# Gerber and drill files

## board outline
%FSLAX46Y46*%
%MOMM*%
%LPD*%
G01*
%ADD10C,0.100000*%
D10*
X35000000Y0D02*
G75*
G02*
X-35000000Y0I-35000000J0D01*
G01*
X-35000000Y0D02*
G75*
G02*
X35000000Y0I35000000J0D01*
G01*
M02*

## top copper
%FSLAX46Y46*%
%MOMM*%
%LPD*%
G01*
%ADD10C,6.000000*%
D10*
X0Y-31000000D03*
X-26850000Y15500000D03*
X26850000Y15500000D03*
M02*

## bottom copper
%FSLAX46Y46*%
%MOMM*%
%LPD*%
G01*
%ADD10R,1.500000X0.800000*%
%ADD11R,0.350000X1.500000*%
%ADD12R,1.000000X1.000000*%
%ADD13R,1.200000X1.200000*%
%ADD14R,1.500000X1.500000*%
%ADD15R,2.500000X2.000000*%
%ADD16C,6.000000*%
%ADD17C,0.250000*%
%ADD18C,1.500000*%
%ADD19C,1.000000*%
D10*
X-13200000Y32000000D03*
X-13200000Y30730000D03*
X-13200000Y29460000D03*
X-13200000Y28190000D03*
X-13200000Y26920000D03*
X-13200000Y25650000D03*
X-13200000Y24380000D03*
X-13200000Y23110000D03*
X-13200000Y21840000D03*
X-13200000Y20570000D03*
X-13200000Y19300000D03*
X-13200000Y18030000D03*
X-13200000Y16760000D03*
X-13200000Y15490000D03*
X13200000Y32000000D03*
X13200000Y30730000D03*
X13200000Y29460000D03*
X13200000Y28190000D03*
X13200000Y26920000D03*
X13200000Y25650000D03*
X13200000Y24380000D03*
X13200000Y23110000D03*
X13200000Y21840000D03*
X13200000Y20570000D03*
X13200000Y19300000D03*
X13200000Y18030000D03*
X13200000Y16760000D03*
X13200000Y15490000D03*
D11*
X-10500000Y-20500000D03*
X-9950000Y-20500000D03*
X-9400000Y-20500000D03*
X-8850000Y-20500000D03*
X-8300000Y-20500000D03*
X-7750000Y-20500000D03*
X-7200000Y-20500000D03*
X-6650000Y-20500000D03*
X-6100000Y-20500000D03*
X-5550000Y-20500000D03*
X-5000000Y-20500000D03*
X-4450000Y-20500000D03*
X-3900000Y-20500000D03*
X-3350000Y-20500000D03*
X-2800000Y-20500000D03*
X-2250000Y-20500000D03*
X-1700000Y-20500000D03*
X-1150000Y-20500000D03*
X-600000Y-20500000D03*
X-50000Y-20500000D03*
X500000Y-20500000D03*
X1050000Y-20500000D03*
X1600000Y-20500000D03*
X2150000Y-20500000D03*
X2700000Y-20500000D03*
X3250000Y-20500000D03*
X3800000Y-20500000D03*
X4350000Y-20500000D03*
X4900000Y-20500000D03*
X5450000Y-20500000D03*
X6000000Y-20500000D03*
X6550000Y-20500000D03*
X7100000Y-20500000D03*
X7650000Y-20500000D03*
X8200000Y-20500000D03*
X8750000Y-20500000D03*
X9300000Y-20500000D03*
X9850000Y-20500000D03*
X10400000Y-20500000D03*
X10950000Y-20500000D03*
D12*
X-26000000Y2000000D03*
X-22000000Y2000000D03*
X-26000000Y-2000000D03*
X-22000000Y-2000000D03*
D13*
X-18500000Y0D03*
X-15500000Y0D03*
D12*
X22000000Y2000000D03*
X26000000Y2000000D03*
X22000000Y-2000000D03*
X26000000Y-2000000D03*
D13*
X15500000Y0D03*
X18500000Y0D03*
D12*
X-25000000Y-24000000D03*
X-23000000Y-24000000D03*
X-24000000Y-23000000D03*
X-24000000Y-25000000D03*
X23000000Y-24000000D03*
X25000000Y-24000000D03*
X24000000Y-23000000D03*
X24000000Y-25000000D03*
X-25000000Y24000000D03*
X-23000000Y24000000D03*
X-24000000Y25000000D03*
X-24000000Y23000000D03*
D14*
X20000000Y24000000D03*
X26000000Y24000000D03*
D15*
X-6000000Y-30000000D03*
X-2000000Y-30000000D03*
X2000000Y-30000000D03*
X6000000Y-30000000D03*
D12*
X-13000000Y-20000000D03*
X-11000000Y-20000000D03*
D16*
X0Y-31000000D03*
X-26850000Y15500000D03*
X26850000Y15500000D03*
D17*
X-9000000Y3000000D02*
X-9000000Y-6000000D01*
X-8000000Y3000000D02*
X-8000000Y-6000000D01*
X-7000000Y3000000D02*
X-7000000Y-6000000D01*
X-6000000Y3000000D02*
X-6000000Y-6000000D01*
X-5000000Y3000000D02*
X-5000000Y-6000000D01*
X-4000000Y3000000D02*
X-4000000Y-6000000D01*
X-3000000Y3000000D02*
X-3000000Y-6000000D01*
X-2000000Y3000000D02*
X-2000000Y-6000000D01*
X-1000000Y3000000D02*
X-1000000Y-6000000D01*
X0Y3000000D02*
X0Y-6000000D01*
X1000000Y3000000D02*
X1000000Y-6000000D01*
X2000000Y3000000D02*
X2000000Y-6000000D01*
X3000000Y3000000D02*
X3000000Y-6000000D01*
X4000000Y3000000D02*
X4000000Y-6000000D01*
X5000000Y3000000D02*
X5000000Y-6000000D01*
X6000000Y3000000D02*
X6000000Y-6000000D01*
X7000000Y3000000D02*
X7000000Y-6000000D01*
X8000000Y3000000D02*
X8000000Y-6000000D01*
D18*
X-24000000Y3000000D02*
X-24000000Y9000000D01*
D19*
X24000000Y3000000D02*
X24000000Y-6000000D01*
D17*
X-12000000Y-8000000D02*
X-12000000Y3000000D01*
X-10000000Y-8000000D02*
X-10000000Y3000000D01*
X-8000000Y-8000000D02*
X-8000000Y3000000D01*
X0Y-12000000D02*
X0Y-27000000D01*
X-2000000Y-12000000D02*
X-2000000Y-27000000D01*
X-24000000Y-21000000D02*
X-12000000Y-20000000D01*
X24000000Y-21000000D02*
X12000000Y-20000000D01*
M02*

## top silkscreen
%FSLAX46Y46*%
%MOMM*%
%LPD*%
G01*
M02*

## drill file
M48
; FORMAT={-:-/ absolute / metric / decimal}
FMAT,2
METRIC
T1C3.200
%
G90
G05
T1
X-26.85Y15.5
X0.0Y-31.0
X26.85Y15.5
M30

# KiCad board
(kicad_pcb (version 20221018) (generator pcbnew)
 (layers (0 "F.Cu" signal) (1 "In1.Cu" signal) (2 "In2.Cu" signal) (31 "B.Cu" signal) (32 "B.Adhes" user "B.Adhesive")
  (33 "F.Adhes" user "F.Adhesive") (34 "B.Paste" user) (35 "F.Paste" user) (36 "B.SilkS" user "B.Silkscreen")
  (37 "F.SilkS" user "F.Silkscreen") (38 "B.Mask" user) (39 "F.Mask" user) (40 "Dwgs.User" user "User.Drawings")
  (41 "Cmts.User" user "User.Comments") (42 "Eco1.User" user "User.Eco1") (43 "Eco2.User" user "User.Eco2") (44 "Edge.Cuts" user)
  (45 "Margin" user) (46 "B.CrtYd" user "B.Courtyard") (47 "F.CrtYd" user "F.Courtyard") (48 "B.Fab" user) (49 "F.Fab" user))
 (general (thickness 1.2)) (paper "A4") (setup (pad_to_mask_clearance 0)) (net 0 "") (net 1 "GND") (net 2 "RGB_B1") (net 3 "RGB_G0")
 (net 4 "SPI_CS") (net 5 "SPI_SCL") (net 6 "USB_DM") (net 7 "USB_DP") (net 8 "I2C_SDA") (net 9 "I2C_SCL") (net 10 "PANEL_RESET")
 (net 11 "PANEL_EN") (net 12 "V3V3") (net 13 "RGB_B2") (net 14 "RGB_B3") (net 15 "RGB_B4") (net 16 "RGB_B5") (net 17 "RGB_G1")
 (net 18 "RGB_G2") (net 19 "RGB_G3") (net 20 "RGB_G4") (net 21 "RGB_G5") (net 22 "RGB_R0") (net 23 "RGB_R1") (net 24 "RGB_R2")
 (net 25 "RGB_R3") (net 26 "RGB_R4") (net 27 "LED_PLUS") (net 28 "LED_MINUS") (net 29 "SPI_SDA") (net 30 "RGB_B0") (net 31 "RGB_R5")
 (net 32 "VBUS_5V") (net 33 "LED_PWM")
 (gr_circle (center 0 0) (end 35 0) (stroke (width 0.1) (type solid)) (fill none) (layer "Edge.Cuts"))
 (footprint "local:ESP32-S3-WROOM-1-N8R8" (layer "B.Cu") (at 0 -12 0)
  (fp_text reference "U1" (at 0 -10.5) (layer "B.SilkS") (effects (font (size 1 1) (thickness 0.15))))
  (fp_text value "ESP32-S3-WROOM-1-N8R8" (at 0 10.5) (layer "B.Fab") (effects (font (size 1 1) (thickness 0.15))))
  (pad "1" smd rect (at -13.2 -20.0) (size 1.5 0.8) (layers "B.Cu" "B.Mask" "B.Paste") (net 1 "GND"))
  (pad "2" smd rect (at -13.2 -18.73) (size 1.5 0.8) (layers "B.Cu" "B.Mask" "B.Paste") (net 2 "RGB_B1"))
  (pad "3" smd rect (at -13.2 -17.46) (size 1.5 0.8) (layers "B.Cu" "B.Mask" "B.Paste") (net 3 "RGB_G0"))
  (pad "4" smd rect (at -13.2 -16.19) (size 1.5 0.8) (layers "B.Cu" "B.Mask" "B.Paste") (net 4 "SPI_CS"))
  (pad "5" smd rect (at -13.2 -14.92) (size 1.5 0.8) (layers "B.Cu" "B.Mask" "B.Paste") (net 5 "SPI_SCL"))
  (pad "6" smd rect (at -13.2 -13.65) (size 1.5 0.8) (layers "B.Cu" "B.Mask" "B.Paste") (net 1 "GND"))
  (pad "7" smd rect (at -13.2 -12.379999999999999) (size 1.5 0.8) (layers "B.Cu" "B.Mask" "B.Paste") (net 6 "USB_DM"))
  (pad "8" smd rect (at -13.2 -11.11) (size 1.5 0.8) (layers "B.Cu" "B.Mask" "B.Paste") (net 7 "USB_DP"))
  (pad "9" smd rect (at -13.2 -9.84) (size 1.5 0.8) (layers "B.Cu" "B.Mask" "B.Paste") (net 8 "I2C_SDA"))
  (pad "10" smd rect (at -13.2 -8.57) (size 1.5 0.8) (layers "B.Cu" "B.Mask" "B.Paste") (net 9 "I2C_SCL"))
  (pad "11" smd rect (at -13.2 -7.300000000000001) (size 1.5 0.8) (layers "B.Cu" "B.Mask" "B.Paste") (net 1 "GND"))
  (pad "12" smd rect (at -13.2 -6.029999999999999) (size 1.5 0.8) (layers "B.Cu" "B.Mask" "B.Paste") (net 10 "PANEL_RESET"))
  (pad "13" smd rect (at -13.2 -4.76) (size 1.5 0.8) (layers "B.Cu" "B.Mask" "B.Paste") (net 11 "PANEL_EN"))
  (pad "14" smd rect (at -13.2 -3.4899999999999984) (size 1.5 0.8) (layers "B.Cu" "B.Mask" "B.Paste") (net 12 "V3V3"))
  (pad "15" smd rect (at 13.2 -20.0) (size 1.5 0.8) (layers "B.Cu" "B.Mask" "B.Paste") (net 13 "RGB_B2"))
  (pad "16" smd rect (at 13.2 -18.73) (size 1.5 0.8) (layers "B.Cu" "B.Mask" "B.Paste") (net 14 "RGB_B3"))
  (pad "17" smd rect (at 13.2 -17.46) (size 1.5 0.8) (layers "B.Cu" "B.Mask" "B.Paste") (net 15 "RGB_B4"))
  (pad "18" smd rect (at 13.2 -16.19) (size 1.5 0.8) (layers "B.Cu" "B.Mask" "B.Paste") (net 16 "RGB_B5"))
  (pad "19" smd rect (at 13.2 -14.92) (size 1.5 0.8) (layers "B.Cu" "B.Mask" "B.Paste") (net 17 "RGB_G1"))
  (pad "20" smd rect (at 13.2 -13.65) (size 1.5 0.8) (layers "B.Cu" "B.Mask" "B.Paste") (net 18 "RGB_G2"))
  (pad "21" smd rect (at 13.2 -12.379999999999999) (size 1.5 0.8) (layers "B.Cu" "B.Mask" "B.Paste") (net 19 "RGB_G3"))
  (pad "22" smd rect (at 13.2 -11.11) (size 1.5 0.8) (layers "B.Cu" "B.Mask" "B.Paste") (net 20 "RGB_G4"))
  (pad "23" smd rect (at 13.2 -9.84) (size 1.5 0.8) (layers "B.Cu" "B.Mask" "B.Paste") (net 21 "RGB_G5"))
  (pad "24" smd rect (at 13.2 -8.57) (size 1.5 0.8) (layers "B.Cu" "B.Mask" "B.Paste") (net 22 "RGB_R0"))
  (pad "25" smd rect (at 13.2 -7.300000000000001) (size 1.5 0.8) (layers "B.Cu" "B.Mask" "B.Paste") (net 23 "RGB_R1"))
  (pad "26" smd rect (at 13.2 -6.029999999999999) (size 1.5 0.8) (layers "B.Cu" "B.Mask" "B.Paste") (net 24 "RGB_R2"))
  (pad "27" smd rect (at 13.2 -4.76) (size 1.5 0.8) (layers "B.Cu" "B.Mask" "B.Paste") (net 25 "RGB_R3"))
  (pad "28" smd rect (at 13.2 -3.4899999999999984) (size 1.5 0.8) (layers "B.Cu" "B.Mask" "B.Paste") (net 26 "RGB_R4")))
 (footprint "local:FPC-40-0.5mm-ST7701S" (layer "B.Cu") (at 0 8 0)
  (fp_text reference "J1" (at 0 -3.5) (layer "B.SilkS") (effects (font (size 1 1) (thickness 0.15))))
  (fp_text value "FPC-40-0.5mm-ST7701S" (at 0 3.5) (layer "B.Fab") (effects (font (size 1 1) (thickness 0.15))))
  (pad "1" smd rect (at -10.5 12.5) (size 0.35 1.5) (layers "B.Cu" "B.Mask" "B.Paste") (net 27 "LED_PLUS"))
  (pad "2" smd rect (at -9.95 12.5) (size 0.35 1.5) (layers "B.Cu" "B.Mask" "B.Paste") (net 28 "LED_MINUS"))
  (pad "3" smd rect (at -9.4 12.5) (size 0.35 1.5) (layers "B.Cu" "B.Mask" "B.Paste") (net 1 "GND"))
  (pad "4" smd rect (at -8.85 12.5) (size 0.35 1.5) (layers "B.Cu" "B.Mask" "B.Paste") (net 12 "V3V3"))
  (pad "5" smd rect (at -8.3 12.5) (size 0.35 1.5) (layers "B.Cu" "B.Mask" "B.Paste") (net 10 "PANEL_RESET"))
  (pad "6" smd rect (at -7.75 12.5) (size 0.35 1.5) (layers "B.Cu" "B.Mask" "B.Paste") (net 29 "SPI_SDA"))
  (pad "7" smd rect (at -7.199999999999999 12.5) (size 0.35 1.5) (layers "B.Cu" "B.Mask" "B.Paste") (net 5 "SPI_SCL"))
  (pad "8" smd rect (at -6.6499999999999995 12.5) (size 0.35 1.5) (layers "B.Cu" "B.Mask" "B.Paste") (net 4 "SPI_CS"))
  (pad "9" smd rect (at -6.1 12.5) (size 0.35 1.5) (layers "B.Cu" "B.Mask" "B.Paste") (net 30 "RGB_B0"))
  (pad "10" smd rect (at -5.55 12.5) (size 0.35 1.5) (layers "B.Cu" "B.Mask" "B.Paste") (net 2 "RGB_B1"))
  (pad "11" smd rect (at -5.0 12.5) (size 0.35 1.5) (layers "B.Cu" "B.Mask" "B.Paste") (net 13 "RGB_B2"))
  (pad "12" smd rect (at -4.449999999999999 12.5) (size 0.35 1.5) (layers "B.Cu" "B.Mask" "B.Paste") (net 14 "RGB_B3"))
  (pad "13" smd rect (at -3.8999999999999995 12.5) (size 0.35 1.5) (layers "B.Cu" "B.Mask" "B.Paste") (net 15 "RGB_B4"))
  (pad "14" smd rect (at -3.3499999999999996 12.5) (size 0.35 1.5) (layers "B.Cu" "B.Mask" "B.Paste") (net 16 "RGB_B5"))
  (pad "15" smd rect (at -2.799999999999999 12.5) (size 0.35 1.5) (layers "B.Cu" "B.Mask" "B.Paste") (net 3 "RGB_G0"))
  (pad "16" smd rect (at -2.25 12.5) (size 0.35 1.5) (layers "B.Cu" "B.Mask" "B.Paste") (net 17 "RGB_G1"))
  (pad "17" smd rect (at -1.6999999999999993 12.5) (size 0.35 1.5) (layers "B.Cu" "B.Mask" "B.Paste") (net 18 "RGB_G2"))
  (pad "18" smd rect (at -1.1499999999999986 12.5) (size 0.35 1.5) (layers "B.Cu" "B.Mask" "B.Paste") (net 19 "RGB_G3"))
  (pad "19" smd rect (at -0.5999999999999996 12.5) (size 0.35 1.5) (layers "B.Cu" "B.Mask" "B.Paste") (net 20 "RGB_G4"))
  (pad "20" smd rect (at -0.049999999999998934 12.5) (size 0.35 1.5) (layers "B.Cu" "B.Mask" "B.Paste") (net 21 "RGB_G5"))
  (pad "21" smd rect (at 0.5 12.5) (size 0.35 1.5) (layers "B.Cu" "B.Mask" "B.Paste") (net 22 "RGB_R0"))
  (pad "22" smd rect (at 1.0500000000000007 12.5) (size 0.35 1.5) (layers "B.Cu" "B.Mask" "B.Paste") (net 23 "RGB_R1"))
  (pad "23" smd rect (at 1.6000000000000014 12.5) (size 0.35 1.5) (layers "B.Cu" "B.Mask" "B.Paste") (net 24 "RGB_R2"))
  (pad "24" smd rect (at 2.1500000000000004 12.5) (size 0.35 1.5) (layers "B.Cu" "B.Mask" "B.Paste") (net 25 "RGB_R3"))
  (pad "25" smd rect (at 2.700000000000001 12.5) (size 0.35 1.5) (layers "B.Cu" "B.Mask" "B.Paste") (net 26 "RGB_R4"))
  (pad "26" smd rect (at 3.2500000000000018 12.5) (size 0.35 1.5) (layers "B.Cu" "B.Mask" "B.Paste") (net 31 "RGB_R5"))
  (pad "27" smd rect (at 3.8000000000000007 12.5) (size 0.35 1.5) (layers "B.Cu" "B.Mask" "B.Paste") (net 1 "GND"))
  (pad "28" smd rect (at 4.350000000000001 12.5) (size 0.35 1.5) (layers "B.Cu" "B.Mask" "B.Paste") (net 1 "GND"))
  (pad "29" smd rect (at 4.900000000000002 12.5) (size 0.35 1.5) (layers "B.Cu" "B.Mask" "B.Paste") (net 1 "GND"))
  (pad "30" smd rect (at 5.450000000000001 12.5) (size 0.35 1.5) (layers "B.Cu" "B.Mask" "B.Paste") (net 1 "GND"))
  (pad "31" smd rect (at 6.0 12.5) (size 0.35 1.5) (layers "B.Cu" "B.Mask" "B.Paste") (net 1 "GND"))
  (pad "32" smd rect (at 6.550000000000001 12.5) (size 0.35 1.5) (layers "B.Cu" "B.Mask" "B.Paste") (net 1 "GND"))
  (pad "33" smd rect (at 7.100000000000001 12.5) (size 0.35 1.5) (layers "B.Cu" "B.Mask" "B.Paste") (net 1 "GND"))
  (pad "34" smd rect (at 7.650000000000002 12.5) (size 0.35 1.5) (layers "B.Cu" "B.Mask" "B.Paste") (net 1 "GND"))
  (pad "35" smd rect (at 8.200000000000003 12.5) (size 0.35 1.5) (layers "B.Cu" "B.Mask" "B.Paste") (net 1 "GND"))
  (pad "36" smd rect (at 8.75 12.5) (size 0.35 1.5) (layers "B.Cu" "B.Mask" "B.Paste") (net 1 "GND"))
  (pad "37" smd rect (at 9.3 12.5) (size 0.35 1.5) (layers "B.Cu" "B.Mask" "B.Paste") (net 1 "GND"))
  (pad "38" smd rect (at 9.850000000000001 12.5) (size 0.35 1.5) (layers "B.Cu" "B.Mask" "B.Paste") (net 1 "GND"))
  (pad "39" smd rect (at 10.400000000000002 12.5) (size 0.35 1.5) (layers "B.Cu" "B.Mask" "B.Paste") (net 1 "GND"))
  (pad "40" smd rect (at 10.950000000000003 12.5) (size 0.35 1.5) (layers "B.Cu" "B.Mask" "B.Paste") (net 1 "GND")))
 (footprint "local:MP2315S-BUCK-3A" (layer "B.Cu") (at -24 0 0)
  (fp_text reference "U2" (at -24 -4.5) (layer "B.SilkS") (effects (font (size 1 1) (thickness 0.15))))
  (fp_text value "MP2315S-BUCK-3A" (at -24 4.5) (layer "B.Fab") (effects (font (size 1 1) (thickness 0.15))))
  (pad "1" smd rect (at -2 -2) (size 1 1) (layers "B.Cu" "B.Mask" "B.Paste") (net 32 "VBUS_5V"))
  (pad "2" smd rect (at 2 -2) (size 1 1) (layers "B.Cu" "B.Mask" "B.Paste") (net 12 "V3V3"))
  (pad "3" smd rect (at -2 2) (size 1 1) (layers "B.Cu" "B.Mask" "B.Paste") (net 1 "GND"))
  (pad "4" smd rect (at 2 2) (size 1 1) (layers "B.Cu" "B.Mask" "B.Paste") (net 12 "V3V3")))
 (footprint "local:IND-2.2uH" (layer "B.Cu") (at -17 0 0)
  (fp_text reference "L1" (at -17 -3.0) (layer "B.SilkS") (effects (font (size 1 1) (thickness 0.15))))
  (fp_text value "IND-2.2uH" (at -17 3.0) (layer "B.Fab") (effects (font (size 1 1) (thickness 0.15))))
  (pad "1" smd rect (at -1.5 0) (size 1.2 1.2) (layers "B.Cu" "B.Mask" "B.Paste") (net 12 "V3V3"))
  (pad "2" smd rect (at 1.5 0) (size 1.2 1.2) (layers "B.Cu" "B.Mask" "B.Paste") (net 12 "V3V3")))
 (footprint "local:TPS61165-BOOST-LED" (layer "B.Cu") (at 24 0 0)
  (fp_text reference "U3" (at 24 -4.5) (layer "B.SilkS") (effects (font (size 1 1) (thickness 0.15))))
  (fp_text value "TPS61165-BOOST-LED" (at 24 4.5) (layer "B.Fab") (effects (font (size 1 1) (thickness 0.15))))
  (pad "1" smd rect (at -2 -2) (size 1 1) (layers "B.Cu" "B.Mask" "B.Paste") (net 32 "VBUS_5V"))
  (pad "2" smd rect (at 2 -2) (size 1 1) (layers "B.Cu" "B.Mask" "B.Paste") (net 27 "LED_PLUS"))
  (pad "3" smd rect (at -2 2) (size 1 1) (layers "B.Cu" "B.Mask" "B.Paste") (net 1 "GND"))
  (pad "4" smd rect (at 2 2) (size 1 1) (layers "B.Cu" "B.Mask" "B.Paste") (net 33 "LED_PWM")))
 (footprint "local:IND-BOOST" (layer "B.Cu") (at 17 0 0)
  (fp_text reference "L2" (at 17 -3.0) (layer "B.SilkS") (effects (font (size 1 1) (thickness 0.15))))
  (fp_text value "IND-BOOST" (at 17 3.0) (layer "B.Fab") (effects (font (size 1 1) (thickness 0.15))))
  (pad "1" smd rect (at -1.5 0) (size 1.2 1.2) (layers "B.Cu" "B.Mask" "B.Paste") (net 32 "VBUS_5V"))
  (pad "2" smd rect (at 1.5 0) (size 1.2 1.2) (layers "B.Cu" "B.Mask" "B.Paste") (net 27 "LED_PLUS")))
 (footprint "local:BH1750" (layer "B.Cu") (at -24 24 0)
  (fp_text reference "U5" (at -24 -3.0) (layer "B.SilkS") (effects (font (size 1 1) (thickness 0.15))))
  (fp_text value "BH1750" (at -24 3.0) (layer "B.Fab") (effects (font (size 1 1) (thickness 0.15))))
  (pad "1" smd rect (at -1 0) (size 1 1) (layers "B.Cu" "B.Mask" "B.Paste") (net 12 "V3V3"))
  (pad "2" smd rect (at 1 0) (size 1 1) (layers "B.Cu" "B.Mask" "B.Paste") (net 8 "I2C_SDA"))
  (pad "3" smd rect (at 0 -1) (size 1 1) (layers "B.Cu" "B.Mask" "B.Paste") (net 9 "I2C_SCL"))
  (pad "4" smd rect (at 0 1) (size 1 1) (layers "B.Cu" "B.Mask" "B.Paste") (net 1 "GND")))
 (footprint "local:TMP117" (layer "B.Cu") (at 24 24 0)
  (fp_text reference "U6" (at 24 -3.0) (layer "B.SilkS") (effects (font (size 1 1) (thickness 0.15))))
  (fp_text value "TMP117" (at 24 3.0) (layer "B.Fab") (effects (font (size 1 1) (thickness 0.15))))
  (pad "1" smd rect (at -1 0) (size 1 1) (layers "B.Cu" "B.Mask" "B.Paste") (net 12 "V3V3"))
  (pad "2" smd rect (at 1 0) (size 1 1) (layers "B.Cu" "B.Mask" "B.Paste") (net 8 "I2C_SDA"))
  (pad "3" smd rect (at 0 -1) (size 1 1) (layers "B.Cu" "B.Mask" "B.Paste") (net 9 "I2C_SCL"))
  (pad "4" smd rect (at 0 1) (size 1 1) (layers "B.Cu" "B.Mask" "B.Paste") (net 1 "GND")))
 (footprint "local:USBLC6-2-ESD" (layer "B.Cu") (at -24 -24 0)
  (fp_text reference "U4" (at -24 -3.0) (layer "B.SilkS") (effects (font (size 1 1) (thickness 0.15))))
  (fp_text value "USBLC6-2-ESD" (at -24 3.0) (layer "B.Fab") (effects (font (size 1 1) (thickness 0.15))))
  (pad "1" smd rect (at -1 0) (size 1 1) (layers "B.Cu" "B.Mask" "B.Paste") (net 6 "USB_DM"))
  (pad "2" smd rect (at 1 0) (size 1 1) (layers "B.Cu" "B.Mask" "B.Paste") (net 7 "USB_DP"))
  (pad "3" smd rect (at 0 -1) (size 1 1) (layers "B.Cu" "B.Mask" "B.Paste") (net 1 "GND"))
  (pad "4" smd rect (at 0 1) (size 1 1) (layers "B.Cu" "B.Mask" "B.Paste") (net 32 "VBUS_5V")))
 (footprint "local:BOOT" (layer "B.Cu") (at 20 -24 0)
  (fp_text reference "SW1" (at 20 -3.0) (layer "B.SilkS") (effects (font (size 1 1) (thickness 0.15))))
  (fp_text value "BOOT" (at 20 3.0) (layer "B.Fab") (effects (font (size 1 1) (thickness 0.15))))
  (pad "1" smd rect (at 0 0) (size 1.5 1.5) (layers "B.Cu" "B.Mask" "B.Paste") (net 1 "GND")))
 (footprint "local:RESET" (layer "B.Cu") (at 26 -24 0)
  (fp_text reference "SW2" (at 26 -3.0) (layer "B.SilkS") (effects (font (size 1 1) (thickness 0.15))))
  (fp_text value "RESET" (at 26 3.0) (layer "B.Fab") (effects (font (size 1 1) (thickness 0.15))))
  (pad "1" smd rect (at 0 0) (size 1.5 1.5) (layers "B.Cu" "B.Mask" "B.Paste") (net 1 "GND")))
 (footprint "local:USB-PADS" (layer "B.Cu") (at 0 30 0)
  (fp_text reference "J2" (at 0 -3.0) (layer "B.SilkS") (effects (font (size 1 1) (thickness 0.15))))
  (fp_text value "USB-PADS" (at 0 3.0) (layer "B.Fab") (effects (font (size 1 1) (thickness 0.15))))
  (pad "1" smd rect (at -6 0) (size 2.5 2) (layers "B.Cu" "B.Mask" "B.Paste") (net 32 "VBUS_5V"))
  (pad "2" smd rect (at -2 0) (size 2.5 2) (layers "B.Cu" "B.Mask" "B.Paste") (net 6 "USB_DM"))
  (pad "3" smd rect (at 2 0) (size 2.5 2) (layers "B.Cu" "B.Mask" "B.Paste") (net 7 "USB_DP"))
  (pad "4" smd rect (at 6 0) (size 2.5 2) (layers "B.Cu" "B.Mask" "B.Paste") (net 1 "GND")))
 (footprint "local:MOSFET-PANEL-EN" (layer "B.Cu") (at -12 20 0)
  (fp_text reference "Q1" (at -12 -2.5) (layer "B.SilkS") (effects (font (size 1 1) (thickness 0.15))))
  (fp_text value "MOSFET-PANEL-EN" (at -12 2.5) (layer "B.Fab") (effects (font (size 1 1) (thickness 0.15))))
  (pad "1" smd rect (at -1 0) (size 1 1) (layers "B.Cu" "B.Mask" "B.Paste") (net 12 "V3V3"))
  (pad "2" smd rect (at 1 0) (size 1 1) (layers "B.Cu" "B.Mask" "B.Paste") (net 11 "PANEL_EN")))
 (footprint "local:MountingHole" (layer "F.Cu") (at 0.0 31.0 0)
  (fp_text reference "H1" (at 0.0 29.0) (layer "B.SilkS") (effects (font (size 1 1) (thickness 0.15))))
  (pad "1" thru_hole circle (at 0 0) (size 6 6) (drill 3.2) (layers "*.Cu" "*.Mask") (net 1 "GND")))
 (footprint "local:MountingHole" (layer "F.Cu") (at -26.85 -15.5 0)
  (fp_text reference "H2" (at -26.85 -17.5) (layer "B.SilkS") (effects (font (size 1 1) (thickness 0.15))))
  (pad "1" thru_hole circle (at 0 0) (size 6 6) (drill 3.2) (layers "*.Cu" "*.Mask") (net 1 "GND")))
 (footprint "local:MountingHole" (layer "F.Cu") (at 26.85 -15.5 0)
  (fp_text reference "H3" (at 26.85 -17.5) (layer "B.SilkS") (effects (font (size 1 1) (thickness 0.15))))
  (pad "1" thru_hole circle (at 0 0) (size 6 6) (drill 3.2) (layers "*.Cu" "*.Mask") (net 1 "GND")))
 (segment (start -9.0 -3) (end -9.0 6) (width 0.25) (layer "B.Cu") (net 30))
 (segment (start -8.0 -3) (end -8.0 6) (width 0.25) (layer "B.Cu") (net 2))
 (segment (start -7.0 -3) (end -7.0 6) (width 0.25) (layer "B.Cu") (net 13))
 (segment (start -6.0 -3) (end -6.0 6) (width 0.25) (layer "B.Cu") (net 14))
 (segment (start -5.0 -3) (end -5.0 6) (width 0.25) (layer "B.Cu") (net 15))
 (segment (start -4.0 -3) (end -4.0 6) (width 0.25) (layer "B.Cu") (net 16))
 (segment (start -3.0 -3) (end -3.0 6) (width 0.25) (layer "B.Cu") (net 3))
 (segment (start -2.0 -3) (end -2.0 6) (width 0.25) (layer "B.Cu") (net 17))
 (segment (start -1.0 -3) (end -1.0 6) (width 0.25) (layer "B.Cu") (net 18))
 (segment (start 0.0 -3) (end 0.0 6) (width 0.25) (layer "B.Cu") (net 19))
 (segment (start 1.0 -3) (end 1.0 6) (width 0.25) (layer "B.Cu") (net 20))
 (segment (start 2.0 -3) (end 2.0 6) (width 0.25) (layer "B.Cu") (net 21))
 (segment (start 3.0 -3) (end 3.0 6) (width 0.25) (layer "B.Cu") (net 22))
 (segment (start 4.0 -3) (end 4.0 6) (width 0.25) (layer "B.Cu") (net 23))
 (segment (start 5.0 -3) (end 5.0 6) (width 0.25) (layer "B.Cu") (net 24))
 (segment (start 6.0 -3) (end 6.0 6) (width 0.25) (layer "B.Cu") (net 25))
 (segment (start 7.0 -3) (end 7.0 6) (width 0.25) (layer "B.Cu") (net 26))
 (segment (start 8.0 -3) (end 8.0 6) (width 0.25) (layer "B.Cu") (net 31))
 (segment (start -24 -3) (end -24 -9) (width 1.5) (layer "B.Cu") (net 32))
 (segment (start 24 -3) (end 24 6) (width 1.0) (layer "B.Cu") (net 27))
 (segment (start -12 8) (end -12 -3) (width 0.25) (layer "B.Cu") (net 4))
 (segment (start -10 8) (end -10 -3) (width 0.25) (layer "B.Cu") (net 5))
 (segment (start -8 8) (end -8 -3) (width 0.25) (layer "B.Cu") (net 29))
 (segment (start 0 12) (end 0 27) (width 0.25) (layer "B.Cu") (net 7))
 (segment (start -2 12) (end -2 27) (width 0.25) (layer "B.Cu") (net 6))
 (segment (start -24 21) (end -12 20) (width 0.25) (layer "B.Cu") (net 8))
 (segment (start 24 21) (end 12 20) (width 0.25) (layer "B.Cu") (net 9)))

